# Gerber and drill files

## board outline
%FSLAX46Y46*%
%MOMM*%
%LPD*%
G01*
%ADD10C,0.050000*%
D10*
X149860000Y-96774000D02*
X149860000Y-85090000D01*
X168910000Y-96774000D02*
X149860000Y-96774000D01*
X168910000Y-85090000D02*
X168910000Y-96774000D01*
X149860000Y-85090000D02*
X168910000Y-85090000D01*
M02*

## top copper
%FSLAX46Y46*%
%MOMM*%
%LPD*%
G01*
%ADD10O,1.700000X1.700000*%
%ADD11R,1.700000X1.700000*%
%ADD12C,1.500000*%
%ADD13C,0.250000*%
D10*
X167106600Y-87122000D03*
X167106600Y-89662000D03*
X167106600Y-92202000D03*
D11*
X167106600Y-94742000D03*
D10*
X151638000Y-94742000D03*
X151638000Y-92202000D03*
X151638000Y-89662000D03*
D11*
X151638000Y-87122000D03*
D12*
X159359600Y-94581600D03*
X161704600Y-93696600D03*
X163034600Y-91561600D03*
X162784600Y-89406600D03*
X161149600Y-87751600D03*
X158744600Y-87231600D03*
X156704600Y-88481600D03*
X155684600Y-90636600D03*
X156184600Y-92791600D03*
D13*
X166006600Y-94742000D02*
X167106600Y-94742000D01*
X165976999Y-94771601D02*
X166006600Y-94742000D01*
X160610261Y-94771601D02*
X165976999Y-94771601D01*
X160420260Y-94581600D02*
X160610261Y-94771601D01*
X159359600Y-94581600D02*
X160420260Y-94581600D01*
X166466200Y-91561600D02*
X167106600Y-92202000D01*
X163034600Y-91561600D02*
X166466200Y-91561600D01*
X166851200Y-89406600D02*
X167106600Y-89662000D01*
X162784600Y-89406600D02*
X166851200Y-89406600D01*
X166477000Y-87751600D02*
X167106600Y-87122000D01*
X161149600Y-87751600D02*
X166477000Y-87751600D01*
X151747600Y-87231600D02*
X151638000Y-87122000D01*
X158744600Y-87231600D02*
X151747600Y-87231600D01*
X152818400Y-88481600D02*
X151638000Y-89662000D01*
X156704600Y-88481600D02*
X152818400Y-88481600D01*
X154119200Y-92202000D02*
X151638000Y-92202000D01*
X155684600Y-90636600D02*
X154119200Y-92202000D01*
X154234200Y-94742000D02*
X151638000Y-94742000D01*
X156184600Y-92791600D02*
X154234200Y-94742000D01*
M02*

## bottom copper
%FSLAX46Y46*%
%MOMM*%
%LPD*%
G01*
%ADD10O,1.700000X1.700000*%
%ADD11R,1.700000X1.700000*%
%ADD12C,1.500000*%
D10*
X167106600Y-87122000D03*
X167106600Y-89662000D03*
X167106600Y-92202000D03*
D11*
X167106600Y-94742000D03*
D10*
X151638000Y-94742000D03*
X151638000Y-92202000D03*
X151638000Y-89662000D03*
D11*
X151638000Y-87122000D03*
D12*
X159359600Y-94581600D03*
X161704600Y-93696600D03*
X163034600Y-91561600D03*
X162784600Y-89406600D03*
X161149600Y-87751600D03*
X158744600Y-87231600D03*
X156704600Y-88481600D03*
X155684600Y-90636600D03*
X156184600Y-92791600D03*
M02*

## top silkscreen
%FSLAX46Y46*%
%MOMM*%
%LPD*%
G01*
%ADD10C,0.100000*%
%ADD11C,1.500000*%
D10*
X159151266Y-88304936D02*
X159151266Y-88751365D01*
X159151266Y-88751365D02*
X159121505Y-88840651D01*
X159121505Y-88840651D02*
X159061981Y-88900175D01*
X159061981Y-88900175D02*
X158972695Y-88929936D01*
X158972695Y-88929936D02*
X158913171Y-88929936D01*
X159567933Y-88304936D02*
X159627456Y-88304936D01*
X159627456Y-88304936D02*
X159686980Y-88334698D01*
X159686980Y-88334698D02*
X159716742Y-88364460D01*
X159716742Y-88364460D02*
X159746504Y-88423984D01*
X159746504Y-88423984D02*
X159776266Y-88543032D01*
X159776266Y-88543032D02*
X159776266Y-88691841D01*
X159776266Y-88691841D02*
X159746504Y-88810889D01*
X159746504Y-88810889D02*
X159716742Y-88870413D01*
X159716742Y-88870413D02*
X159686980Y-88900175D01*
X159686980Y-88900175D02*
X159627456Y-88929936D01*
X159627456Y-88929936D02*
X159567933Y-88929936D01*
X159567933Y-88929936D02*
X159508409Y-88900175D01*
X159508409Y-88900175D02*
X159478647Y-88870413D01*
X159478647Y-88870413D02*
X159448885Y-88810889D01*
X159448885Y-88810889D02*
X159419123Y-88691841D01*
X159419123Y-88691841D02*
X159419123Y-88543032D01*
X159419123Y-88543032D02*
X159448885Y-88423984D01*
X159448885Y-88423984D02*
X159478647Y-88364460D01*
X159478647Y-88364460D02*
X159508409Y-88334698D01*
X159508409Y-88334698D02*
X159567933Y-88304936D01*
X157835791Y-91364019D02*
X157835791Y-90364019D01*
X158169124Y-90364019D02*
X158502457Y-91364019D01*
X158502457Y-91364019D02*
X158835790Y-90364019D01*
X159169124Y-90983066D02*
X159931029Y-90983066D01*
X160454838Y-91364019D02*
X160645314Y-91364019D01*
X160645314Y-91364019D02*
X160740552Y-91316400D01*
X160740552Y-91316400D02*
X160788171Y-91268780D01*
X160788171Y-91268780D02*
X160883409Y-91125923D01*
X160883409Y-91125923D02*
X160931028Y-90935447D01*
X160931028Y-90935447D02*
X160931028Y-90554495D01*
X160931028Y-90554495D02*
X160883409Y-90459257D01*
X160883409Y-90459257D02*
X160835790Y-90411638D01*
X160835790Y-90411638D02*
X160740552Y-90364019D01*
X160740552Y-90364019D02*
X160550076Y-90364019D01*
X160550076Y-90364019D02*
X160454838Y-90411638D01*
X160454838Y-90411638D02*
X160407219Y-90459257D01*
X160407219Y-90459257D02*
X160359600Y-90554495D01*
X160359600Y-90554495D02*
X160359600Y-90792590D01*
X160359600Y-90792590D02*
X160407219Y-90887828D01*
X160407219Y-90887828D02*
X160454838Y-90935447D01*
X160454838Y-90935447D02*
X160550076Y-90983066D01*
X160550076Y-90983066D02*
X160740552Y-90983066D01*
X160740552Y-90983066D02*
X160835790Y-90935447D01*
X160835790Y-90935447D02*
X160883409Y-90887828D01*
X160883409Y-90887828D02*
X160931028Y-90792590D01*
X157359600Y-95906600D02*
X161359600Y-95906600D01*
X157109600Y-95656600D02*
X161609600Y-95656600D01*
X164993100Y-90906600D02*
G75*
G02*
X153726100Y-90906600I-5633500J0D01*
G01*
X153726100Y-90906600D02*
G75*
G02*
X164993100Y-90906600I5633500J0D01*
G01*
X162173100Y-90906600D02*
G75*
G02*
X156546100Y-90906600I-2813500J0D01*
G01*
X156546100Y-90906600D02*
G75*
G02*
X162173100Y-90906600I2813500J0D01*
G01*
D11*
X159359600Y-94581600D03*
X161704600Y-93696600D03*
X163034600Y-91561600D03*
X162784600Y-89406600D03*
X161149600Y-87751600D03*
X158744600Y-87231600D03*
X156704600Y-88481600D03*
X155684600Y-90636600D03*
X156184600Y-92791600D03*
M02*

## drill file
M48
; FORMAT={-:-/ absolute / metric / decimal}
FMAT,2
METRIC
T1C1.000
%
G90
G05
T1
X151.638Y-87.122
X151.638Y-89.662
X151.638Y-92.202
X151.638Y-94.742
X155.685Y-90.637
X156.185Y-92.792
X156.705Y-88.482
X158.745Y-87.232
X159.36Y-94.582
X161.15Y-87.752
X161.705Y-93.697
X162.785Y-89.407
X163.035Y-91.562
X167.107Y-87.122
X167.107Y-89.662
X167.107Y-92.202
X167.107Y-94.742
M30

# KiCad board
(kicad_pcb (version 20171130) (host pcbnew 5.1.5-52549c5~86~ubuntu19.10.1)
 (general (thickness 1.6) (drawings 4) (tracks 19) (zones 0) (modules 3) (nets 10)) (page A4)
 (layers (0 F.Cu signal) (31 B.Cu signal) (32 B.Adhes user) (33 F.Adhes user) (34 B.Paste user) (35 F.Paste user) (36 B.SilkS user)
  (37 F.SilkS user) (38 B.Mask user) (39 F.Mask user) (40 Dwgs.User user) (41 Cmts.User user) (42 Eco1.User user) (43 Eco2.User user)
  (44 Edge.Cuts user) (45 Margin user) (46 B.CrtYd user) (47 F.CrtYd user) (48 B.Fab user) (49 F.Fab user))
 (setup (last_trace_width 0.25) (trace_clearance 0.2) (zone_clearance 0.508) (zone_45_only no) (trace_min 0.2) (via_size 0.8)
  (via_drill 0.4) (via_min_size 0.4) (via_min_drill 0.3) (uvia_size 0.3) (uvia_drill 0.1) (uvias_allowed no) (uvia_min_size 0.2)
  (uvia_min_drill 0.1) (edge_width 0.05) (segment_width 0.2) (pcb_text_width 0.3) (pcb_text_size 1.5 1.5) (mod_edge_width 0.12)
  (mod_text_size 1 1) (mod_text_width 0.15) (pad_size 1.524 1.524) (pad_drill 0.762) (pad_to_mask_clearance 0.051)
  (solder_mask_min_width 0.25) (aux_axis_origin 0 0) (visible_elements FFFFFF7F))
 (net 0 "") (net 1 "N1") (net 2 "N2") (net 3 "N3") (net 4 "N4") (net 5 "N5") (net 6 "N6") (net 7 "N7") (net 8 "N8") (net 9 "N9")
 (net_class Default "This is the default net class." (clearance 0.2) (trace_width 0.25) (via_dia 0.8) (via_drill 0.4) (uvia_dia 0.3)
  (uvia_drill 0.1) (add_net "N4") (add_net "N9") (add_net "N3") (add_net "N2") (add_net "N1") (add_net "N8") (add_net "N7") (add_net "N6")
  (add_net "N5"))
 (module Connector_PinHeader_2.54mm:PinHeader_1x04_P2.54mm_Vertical (layer B.Cu) (at 167.1066 94.742)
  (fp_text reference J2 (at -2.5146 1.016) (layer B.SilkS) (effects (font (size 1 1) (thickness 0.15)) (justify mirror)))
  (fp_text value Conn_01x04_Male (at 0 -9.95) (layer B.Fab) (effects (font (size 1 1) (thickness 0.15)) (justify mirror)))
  (pad 4 thru_hole oval (at 0 -7.62) (size 1.7 1.7) (drill 1) (layers *.Cu *.Mask) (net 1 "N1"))
  (pad 3 thru_hole oval (at 0 -5.08) (size 1.7 1.7) (drill 1) (layers *.Cu *.Mask) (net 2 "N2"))
  (pad 2 thru_hole oval (at 0 -2.54) (size 1.7 1.7) (drill 1) (layers *.Cu *.Mask) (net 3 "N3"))
  (pad 1 thru_hole rect (at 0 0) (size 1.7 1.7) (drill 1) (layers *.Cu *.Mask) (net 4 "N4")))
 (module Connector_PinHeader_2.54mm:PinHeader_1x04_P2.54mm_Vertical (layer B.Cu) (at 151.638 87.122 180)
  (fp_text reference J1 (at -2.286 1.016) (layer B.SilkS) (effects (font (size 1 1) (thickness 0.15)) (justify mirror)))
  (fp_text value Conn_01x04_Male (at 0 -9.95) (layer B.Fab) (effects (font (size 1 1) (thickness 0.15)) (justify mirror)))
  (pad 4 thru_hole oval (at 0 -7.62 180) (size 1.7 1.7) (drill 1) (layers *.Cu *.Mask) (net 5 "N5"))
  (pad 3 thru_hole oval (at 0 -5.08 180) (size 1.7 1.7) (drill 1) (layers *.Cu *.Mask) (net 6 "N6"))
  (pad 2 thru_hole oval (at 0 -2.54 180) (size 1.7 1.7) (drill 1) (layers *.Cu *.Mask) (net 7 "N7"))
  (pad 1 thru_hole rect (at 0 0 180) (size 1.7 1.7) (drill 1) (layers *.Cu *.Mask) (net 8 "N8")))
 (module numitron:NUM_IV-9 (layer F.Cu) (at 159.3596 90.9066)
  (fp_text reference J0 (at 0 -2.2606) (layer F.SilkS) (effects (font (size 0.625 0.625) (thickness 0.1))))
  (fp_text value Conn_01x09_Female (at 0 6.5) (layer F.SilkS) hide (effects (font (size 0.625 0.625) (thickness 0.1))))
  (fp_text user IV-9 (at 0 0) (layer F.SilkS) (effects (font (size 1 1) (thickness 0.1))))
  (fp_line (start -2 5) (end 2 5) (layer F.SilkS) (width 0.1))
  (fp_line (start -2.25 4.75) (end 2.25 4.75) (layer F.SilkS) (width 0.1))
  (fp_circle (center 0 0) (end 3.983486 3.983486) (layer F.SilkS) (width 0.1))
  (fp_circle (center 0 0) (end 1.989445 1.989445) (layer F.SilkS) (width 0.1))
  (pad 1 thru_hole circle (at 0 3.675) (size 1.5 1.5) (drill 1) (layers *.Cu *.Mask F.SilkS) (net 4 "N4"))
  (pad 2 thru_hole circle (at 2.345 2.79) (size 1.5 1.5) (drill 1) (layers *.Cu *.Mask F.SilkS) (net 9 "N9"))
  (pad 3 thru_hole circle (at 3.675 0.655) (size 1.5 1.5) (drill 1) (layers *.Cu *.Mask F.SilkS) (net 3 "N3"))
  (pad 4 thru_hole circle (at 3.425 -1.5) (size 1.5 1.5) (drill 1) (layers *.Cu *.Mask F.SilkS) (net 2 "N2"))
  (pad 5 thru_hole circle (at 1.79 -3.155) (size 1.5 1.5) (drill 1) (layers *.Cu *.Mask F.SilkS) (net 1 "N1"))
  (pad 6 thru_hole circle (at -0.615 -3.675) (size 1.5 1.5) (drill 1) (layers *.Cu *.Mask F.SilkS) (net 8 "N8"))
  (pad 7 thru_hole circle (at -2.655 -2.425) (size 1.5 1.5) (drill 1) (layers *.Cu *.Mask F.SilkS) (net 7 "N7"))
  (pad 8 thru_hole circle (at -3.675 -0.27) (size 1.5 1.5) (drill 1) (layers *.Cu *.Mask F.SilkS) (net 6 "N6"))
  (pad 9 thru_hole circle (at -3.175 1.885) (size 1.5 1.5) (drill 1) (layers *.Cu *.Mask F.SilkS) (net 5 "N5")))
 (gr_line (start 149.86 96.774) (end 149.86 85.09) (layer Edge.Cuts) (width 0.05))
 (gr_line (start 168.91 96.774) (end 149.86 96.774) (layer Edge.Cuts) (width 0.05))
 (gr_line (start 168.91 85.09) (end 168.91 96.774) (layer Edge.Cuts) (width 0.05))
 (gr_line (start 149.86 85.09) (end 168.91 85.09) (layer Edge.Cuts) (width 0.05))
 (segment (start 166.0066 94.742) (end 167.1066 94.742) (width 0.25) (layer F.Cu) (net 4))
 (segment (start 165.976999 94.771601) (end 166.0066 94.742) (width 0.25) (layer F.Cu) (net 4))
 (segment (start 160.610261 94.771601) (end 165.976999 94.771601) (width 0.25) (layer F.Cu) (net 4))
 (segment (start 160.42026 94.5816) (end 160.610261 94.771601) (width 0.25) (layer F.Cu) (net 4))
 (segment (start 159.3596 94.5816) (end 160.42026 94.5816) (width 0.25) (layer F.Cu) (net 4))
 (segment (start 166.4662 91.5616) (end 167.1066 92.202) (width 0.25) (layer F.Cu) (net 3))
 (segment (start 163.0346 91.5616) (end 166.4662 91.5616) (width 0.25) (layer F.Cu) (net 3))
 (segment (start 166.8512 89.4066) (end 167.1066 89.662) (width 0.25) (layer F.Cu) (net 2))
 (segment (start 162.7846 89.4066) (end 166.8512 89.4066) (width 0.25) (layer F.Cu) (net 2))
 (segment (start 166.477 87.7516) (end 167.1066 87.122) (width 0.25) (layer F.Cu) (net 1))
 (segment (start 161.1496 87.7516) (end 166.477 87.7516) (width 0.25) (layer F.Cu) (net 1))
 (segment (start 151.7476 87.2316) (end 151.638 87.122) (width 0.25) (layer F.Cu) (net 8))
 (segment (start 158.7446 87.2316) (end 151.7476 87.2316) (width 0.25) (layer F.Cu) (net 8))
 (segment (start 152.8184 88.4816) (end 151.638 89.662) (width 0.25) (layer F.Cu) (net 7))
 (segment (start 156.7046 88.4816) (end 152.8184 88.4816) (width 0.25) (layer F.Cu) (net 7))
 (segment (start 154.1192 92.202) (end 151.638 92.202) (width 0.25) (layer F.Cu) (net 6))
 (segment (start 155.6846 90.6366) (end 154.1192 92.202) (width 0.25) (layer F.Cu) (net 6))
 (segment (start 154.2342 94.742) (end 151.638 94.742) (width 0.25) (layer F.Cu) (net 5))
 (segment (start 156.1846 92.7916) (end 154.2342 94.742) (width 0.25) (layer F.Cu) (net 5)))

